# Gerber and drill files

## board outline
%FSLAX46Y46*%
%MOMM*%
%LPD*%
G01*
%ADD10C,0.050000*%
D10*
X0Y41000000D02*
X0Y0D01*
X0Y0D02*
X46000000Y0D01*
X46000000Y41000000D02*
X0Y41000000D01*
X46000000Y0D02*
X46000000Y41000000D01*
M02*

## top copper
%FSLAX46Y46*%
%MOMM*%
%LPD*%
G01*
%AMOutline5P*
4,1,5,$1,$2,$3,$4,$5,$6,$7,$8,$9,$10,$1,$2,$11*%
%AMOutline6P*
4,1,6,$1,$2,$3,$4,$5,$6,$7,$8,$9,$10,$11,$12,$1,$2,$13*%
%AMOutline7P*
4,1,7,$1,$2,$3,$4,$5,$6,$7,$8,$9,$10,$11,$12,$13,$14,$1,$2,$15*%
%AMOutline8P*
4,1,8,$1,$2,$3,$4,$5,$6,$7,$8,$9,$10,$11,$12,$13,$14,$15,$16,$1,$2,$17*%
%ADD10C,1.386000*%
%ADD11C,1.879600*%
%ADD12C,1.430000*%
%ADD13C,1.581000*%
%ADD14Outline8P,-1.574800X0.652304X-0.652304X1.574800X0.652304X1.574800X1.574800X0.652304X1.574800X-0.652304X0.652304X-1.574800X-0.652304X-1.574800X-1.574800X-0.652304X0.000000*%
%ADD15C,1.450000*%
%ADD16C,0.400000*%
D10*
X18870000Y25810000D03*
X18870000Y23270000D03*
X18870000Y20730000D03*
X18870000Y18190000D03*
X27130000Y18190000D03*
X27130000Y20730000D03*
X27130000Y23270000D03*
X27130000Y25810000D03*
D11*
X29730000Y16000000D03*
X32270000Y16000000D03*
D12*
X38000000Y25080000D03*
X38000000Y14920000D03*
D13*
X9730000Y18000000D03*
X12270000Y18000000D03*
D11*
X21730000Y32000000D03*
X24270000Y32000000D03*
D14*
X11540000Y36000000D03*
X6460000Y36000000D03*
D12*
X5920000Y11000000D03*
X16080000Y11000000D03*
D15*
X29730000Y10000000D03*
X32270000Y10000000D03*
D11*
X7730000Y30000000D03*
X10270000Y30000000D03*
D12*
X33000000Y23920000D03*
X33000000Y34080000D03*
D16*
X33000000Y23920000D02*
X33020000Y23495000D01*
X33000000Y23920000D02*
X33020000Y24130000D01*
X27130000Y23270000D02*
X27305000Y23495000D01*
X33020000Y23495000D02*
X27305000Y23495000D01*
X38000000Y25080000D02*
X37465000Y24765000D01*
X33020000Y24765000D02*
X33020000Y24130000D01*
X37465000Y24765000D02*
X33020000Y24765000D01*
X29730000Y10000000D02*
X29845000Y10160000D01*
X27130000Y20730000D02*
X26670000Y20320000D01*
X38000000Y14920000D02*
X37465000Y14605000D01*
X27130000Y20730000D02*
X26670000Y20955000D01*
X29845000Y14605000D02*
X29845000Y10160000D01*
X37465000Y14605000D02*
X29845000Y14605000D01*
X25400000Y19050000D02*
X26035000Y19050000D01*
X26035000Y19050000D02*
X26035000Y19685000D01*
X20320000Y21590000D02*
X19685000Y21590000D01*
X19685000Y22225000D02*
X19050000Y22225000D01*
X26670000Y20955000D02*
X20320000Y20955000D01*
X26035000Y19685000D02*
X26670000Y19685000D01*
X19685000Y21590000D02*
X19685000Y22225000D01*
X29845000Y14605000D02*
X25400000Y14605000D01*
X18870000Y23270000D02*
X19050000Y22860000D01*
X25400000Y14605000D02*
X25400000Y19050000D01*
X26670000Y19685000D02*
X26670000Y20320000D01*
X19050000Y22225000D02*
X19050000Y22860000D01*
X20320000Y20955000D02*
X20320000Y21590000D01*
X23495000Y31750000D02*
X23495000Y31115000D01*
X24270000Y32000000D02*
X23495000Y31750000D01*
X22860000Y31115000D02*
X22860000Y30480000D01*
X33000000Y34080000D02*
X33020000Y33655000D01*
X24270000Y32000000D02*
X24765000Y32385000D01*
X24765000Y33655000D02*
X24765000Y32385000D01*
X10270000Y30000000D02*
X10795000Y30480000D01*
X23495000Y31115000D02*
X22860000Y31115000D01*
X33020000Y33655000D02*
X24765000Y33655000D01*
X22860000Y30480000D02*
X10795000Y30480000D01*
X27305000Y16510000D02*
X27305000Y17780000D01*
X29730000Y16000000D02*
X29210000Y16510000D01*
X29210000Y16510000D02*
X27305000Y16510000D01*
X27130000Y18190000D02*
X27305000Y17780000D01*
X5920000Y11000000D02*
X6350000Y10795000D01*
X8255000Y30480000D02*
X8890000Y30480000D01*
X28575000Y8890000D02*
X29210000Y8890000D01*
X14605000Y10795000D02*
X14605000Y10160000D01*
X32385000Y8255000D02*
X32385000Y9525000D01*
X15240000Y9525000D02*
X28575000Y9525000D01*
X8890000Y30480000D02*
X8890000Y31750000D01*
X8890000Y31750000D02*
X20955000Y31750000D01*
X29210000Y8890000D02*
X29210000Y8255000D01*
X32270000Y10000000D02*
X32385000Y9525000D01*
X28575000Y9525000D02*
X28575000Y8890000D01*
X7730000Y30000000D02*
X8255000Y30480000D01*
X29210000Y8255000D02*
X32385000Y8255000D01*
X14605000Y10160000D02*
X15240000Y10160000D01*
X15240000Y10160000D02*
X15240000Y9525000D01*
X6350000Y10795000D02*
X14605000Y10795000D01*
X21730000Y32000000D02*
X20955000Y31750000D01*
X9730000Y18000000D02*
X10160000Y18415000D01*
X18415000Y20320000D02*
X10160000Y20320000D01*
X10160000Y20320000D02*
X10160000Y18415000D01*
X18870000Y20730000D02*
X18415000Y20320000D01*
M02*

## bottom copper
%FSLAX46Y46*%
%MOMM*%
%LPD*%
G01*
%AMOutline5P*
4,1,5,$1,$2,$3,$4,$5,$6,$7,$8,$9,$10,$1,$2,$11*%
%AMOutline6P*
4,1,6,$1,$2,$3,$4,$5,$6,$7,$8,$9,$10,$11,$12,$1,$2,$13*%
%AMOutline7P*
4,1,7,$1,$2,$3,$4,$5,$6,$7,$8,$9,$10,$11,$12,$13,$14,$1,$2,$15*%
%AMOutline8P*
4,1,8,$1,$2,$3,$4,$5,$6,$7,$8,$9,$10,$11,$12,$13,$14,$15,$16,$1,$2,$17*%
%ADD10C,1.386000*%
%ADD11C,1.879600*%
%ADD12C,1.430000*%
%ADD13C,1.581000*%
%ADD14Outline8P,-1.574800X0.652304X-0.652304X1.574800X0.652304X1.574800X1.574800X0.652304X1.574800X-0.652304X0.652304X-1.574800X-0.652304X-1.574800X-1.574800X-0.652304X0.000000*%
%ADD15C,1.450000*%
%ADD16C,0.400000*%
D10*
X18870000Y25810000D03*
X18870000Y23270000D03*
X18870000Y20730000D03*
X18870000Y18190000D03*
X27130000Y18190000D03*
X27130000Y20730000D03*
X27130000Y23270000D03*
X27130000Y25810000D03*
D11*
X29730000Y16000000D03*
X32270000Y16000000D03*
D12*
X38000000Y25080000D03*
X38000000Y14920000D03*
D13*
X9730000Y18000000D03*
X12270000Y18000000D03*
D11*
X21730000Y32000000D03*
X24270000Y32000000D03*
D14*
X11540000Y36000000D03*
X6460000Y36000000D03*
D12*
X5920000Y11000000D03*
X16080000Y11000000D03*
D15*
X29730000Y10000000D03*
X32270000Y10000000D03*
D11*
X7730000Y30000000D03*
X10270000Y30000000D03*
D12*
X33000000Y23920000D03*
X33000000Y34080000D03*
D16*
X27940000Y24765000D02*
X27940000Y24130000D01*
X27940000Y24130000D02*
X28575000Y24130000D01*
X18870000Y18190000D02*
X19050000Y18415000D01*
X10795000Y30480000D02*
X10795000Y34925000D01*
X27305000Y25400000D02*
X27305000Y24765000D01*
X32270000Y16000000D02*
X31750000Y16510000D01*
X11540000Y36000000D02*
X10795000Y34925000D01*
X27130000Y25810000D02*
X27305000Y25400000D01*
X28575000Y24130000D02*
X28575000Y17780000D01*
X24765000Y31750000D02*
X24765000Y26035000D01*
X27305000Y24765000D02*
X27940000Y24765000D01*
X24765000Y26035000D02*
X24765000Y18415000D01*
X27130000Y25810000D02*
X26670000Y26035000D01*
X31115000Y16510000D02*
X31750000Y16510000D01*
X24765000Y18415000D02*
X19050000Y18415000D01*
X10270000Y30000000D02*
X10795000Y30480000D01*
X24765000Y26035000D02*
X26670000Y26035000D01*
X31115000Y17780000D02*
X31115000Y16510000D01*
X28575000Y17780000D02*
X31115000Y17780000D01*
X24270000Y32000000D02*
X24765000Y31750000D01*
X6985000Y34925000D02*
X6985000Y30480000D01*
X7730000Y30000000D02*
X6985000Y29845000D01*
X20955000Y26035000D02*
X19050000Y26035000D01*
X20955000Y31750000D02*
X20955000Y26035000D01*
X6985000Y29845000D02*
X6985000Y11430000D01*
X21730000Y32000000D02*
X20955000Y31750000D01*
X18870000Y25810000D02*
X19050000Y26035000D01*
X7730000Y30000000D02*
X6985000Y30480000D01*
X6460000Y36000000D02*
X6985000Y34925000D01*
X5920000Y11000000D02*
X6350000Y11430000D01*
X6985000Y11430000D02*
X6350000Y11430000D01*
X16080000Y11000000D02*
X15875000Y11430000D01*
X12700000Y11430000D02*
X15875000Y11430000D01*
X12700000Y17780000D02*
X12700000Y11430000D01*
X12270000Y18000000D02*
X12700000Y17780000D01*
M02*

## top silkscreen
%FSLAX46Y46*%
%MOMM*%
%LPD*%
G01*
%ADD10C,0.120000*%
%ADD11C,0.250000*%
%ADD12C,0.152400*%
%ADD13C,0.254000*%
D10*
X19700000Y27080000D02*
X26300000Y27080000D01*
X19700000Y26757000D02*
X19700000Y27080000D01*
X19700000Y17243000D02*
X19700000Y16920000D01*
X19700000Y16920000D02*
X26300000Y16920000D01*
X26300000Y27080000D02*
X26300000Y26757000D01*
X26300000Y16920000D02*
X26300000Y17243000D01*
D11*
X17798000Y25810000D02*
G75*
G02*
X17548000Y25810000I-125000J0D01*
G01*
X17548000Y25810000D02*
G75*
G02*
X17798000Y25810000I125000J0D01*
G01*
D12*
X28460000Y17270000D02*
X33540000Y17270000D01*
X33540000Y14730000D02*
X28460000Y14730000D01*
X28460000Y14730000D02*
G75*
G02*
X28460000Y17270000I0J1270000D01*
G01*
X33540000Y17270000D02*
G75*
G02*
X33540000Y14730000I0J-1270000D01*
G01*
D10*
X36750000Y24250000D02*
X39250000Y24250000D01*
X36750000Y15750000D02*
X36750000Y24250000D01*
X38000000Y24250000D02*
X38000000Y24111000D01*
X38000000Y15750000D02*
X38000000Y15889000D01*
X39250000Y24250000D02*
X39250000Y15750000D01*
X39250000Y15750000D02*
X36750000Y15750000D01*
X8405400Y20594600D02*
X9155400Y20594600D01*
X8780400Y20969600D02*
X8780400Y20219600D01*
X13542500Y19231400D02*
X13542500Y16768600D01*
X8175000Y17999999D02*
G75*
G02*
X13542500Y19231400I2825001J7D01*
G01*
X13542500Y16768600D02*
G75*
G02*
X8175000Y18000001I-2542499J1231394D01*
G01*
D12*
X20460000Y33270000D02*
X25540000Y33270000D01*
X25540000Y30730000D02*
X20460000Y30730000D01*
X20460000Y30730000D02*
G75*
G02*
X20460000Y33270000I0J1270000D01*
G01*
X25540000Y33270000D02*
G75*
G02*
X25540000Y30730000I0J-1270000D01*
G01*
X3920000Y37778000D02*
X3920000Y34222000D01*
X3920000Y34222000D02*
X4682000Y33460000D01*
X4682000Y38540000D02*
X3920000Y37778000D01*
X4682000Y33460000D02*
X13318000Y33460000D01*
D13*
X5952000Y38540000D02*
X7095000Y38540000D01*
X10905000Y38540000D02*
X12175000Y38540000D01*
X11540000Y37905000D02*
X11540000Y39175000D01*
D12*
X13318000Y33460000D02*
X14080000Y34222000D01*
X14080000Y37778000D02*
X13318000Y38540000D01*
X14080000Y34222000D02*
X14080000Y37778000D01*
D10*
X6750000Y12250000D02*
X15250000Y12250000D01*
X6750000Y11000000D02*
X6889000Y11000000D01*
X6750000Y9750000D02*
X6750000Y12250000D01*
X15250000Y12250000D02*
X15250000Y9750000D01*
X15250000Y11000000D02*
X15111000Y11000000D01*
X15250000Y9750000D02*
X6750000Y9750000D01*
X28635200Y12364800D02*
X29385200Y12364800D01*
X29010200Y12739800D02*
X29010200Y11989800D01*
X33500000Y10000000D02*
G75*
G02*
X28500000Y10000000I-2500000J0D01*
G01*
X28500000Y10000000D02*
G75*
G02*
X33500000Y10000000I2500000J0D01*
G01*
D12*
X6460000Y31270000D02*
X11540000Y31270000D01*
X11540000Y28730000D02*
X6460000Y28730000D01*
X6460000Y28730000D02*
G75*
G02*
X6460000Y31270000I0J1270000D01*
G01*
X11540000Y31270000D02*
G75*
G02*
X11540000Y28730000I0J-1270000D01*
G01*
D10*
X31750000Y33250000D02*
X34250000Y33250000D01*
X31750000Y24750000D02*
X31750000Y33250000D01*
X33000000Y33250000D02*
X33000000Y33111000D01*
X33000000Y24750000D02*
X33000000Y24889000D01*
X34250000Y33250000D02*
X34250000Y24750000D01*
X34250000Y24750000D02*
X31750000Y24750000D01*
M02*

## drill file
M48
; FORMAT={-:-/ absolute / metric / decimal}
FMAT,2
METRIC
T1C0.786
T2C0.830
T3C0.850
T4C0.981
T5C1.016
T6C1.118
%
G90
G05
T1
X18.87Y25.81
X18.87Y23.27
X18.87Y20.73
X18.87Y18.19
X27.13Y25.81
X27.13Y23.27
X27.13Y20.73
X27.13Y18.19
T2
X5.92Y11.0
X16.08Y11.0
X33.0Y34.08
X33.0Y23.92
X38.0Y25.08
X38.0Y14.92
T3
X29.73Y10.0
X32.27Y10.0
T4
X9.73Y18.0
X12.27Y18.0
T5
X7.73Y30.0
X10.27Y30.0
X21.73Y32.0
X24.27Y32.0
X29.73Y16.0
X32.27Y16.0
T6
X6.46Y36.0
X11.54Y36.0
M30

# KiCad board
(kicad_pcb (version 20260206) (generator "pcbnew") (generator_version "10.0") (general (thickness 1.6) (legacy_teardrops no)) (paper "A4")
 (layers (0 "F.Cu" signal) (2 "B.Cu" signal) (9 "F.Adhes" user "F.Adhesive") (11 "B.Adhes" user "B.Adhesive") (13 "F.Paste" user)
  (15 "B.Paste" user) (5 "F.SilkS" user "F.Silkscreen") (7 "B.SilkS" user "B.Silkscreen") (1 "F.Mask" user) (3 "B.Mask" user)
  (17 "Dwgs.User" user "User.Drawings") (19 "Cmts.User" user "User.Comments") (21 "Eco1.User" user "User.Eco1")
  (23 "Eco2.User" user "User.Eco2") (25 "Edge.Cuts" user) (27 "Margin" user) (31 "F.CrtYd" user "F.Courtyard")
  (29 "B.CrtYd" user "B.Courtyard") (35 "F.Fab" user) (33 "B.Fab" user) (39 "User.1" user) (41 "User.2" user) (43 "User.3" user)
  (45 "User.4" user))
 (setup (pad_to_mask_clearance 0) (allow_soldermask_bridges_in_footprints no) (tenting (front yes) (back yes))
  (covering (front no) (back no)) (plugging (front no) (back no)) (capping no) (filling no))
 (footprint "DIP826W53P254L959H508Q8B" (layer "F.Cu") (at 23 -22)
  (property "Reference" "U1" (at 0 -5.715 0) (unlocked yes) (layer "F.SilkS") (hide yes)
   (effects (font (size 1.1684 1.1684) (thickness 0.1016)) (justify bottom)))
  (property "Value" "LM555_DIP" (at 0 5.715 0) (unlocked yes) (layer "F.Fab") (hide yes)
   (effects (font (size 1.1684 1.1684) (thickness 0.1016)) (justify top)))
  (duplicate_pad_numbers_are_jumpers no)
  (fp_line (start -3.3 -5.08) (end 3.3 -5.08) (stroke (width 0.12) (type solid)) (layer "F.SilkS"))
  (fp_line (start -3.3 -4.757) (end -3.3 -5.08) (stroke (width 0.12) (type solid)) (layer "F.SilkS"))
  (fp_line (start -3.3 4.757) (end -3.3 5.08) (stroke (width 0.12) (type solid)) (layer "F.SilkS"))
  (fp_line (start -3.3 5.08) (end 3.3 5.08) (stroke (width 0.12) (type solid)) (layer "F.SilkS"))
  (fp_line (start 3.3 -5.08) (end 3.3 -4.757) (stroke (width 0.12) (type solid)) (layer "F.SilkS"))
  (fp_line (start 3.3 5.08) (end 3.3 4.757) (stroke (width 0.12) (type solid)) (layer "F.SilkS"))
  (fp_circle (center -5.327 -3.81) (end -5.202 -3.81) (stroke (width 0.25) (type solid)) (fill yes) (layer "F.SilkS"))
  (pad "1" thru_hole circle (at -4.13 -3.81) (size 1.386 1.386) (drill 0.786) (layers "*.Cu" "*.Mask") (remove_unused_layers no) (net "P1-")
   (solder_mask_margin 0.1016) (thermal_bridge_angle 0))
  (pad "2" thru_hole circle (at -4.13 -1.27) (size 1.386 1.386) (drill 0.786) (layers "*.Cu" "*.Mask") (remove_unused_layers no)
   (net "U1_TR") (solder_mask_margin 0.1016) (thermal_bridge_angle 0))
  (pad "3" thru_hole circle (at -4.13 1.27) (size 1.386 1.386) (drill 0.786) (layers "*.Cu" "*.Mask") (remove_unused_layers no)
   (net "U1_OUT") (solder_mask_margin 0.1016) (thermal_bridge_angle 0))
  (pad "4" thru_hole circle (at -4.13 3.81) (size 1.386 1.386) (drill 0.786) (layers "*.Cu" "*.Mask") (remove_unused_layers no) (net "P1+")
   (solder_mask_margin 0.1016) (thermal_bridge_angle 0))
  (pad "5" thru_hole circle (at 4.13 3.81) (size 1.386 1.386) (drill 0.786) (layers "*.Cu" "*.Mask") (remove_unused_layers no) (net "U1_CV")
   (solder_mask_margin 0.1016) (thermal_bridge_angle 0))
  (pad "6" thru_hole circle (at 4.13 1.27) (size 1.386 1.386) (drill 0.786) (layers "*.Cu" "*.Mask") (remove_unused_layers no) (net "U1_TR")
   (solder_mask_margin 0.1016) (thermal_bridge_angle 0))
  (pad "7" thru_hole circle (at 4.13 -1.27) (size 1.386 1.386) (drill 0.786) (layers "*.Cu" "*.Mask") (remove_unused_layers no)
   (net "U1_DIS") (solder_mask_margin 0.1016) (thermal_bridge_angle 0))
  (pad "8" thru_hole circle (at 4.13 -3.81) (size 1.386 1.386) (drill 0.786) (layers "*.Cu" "*.Mask") (remove_unused_layers no) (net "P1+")
   (solder_mask_margin 0.1016) (thermal_bridge_angle 0)))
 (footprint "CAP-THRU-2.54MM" (layer "F.Cu") (at 31 -16)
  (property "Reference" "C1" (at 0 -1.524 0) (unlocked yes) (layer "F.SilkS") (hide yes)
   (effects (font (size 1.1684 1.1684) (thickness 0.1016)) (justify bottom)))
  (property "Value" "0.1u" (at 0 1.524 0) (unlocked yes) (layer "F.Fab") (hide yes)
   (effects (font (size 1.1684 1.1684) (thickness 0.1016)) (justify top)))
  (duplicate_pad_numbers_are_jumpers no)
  (fp_line (start -2.54 -1.27) (end 2.54 -1.27) (stroke (width 0.1524) (type solid)) (layer "F.SilkS"))
  (fp_line (start 2.54 1.27) (end -2.54 1.27) (stroke (width 0.1524) (type solid)) (layer "F.SilkS"))
  (fp_arc (start -2.54 1.27) (mid -3.81 0) (end -2.54 -1.27) (stroke (width 0.1524) (type solid)) (layer "F.SilkS"))
  (fp_arc (start 2.54 -1.27) (mid 3.81 0) (end 2.54 1.27) (stroke (width 0.1524) (type solid)) (layer "F.SilkS"))
  (pad "1" thru_hole circle (at -1.27 0) (size 1.8796 1.8796) (drill 1.016) (layers "*.Cu" "*.Mask") (remove_unused_layers no) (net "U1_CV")
   (solder_mask_margin 0.1016) (thermal_bridge_angle 0))
  (pad "2" thru_hole circle (at 1.27 0) (size 1.8796 1.8796) (drill 1.016) (layers "*.Cu" "*.Mask") (remove_unused_layers no) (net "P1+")
   (solder_mask_margin 0.1016) (thermal_bridge_angle 0)))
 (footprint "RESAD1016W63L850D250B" (layer "F.Cu") (at 38 -20 -90)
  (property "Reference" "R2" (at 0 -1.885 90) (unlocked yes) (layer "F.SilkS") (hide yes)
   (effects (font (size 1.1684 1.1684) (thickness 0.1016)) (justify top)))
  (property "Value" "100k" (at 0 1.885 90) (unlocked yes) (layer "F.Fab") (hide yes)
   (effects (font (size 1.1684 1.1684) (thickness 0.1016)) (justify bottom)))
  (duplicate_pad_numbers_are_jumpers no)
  (fp_line (start -4.25 1.25) (end -4.25 -1.25) (stroke (width 0.12) (type solid)) (layer "F.SilkS"))
  (fp_line (start 4.25 1.25) (end -4.25 1.25) (stroke (width 0.12) (type solid)) (layer "F.SilkS"))
  (fp_line (start -4.25 0) (end -4.111 0) (stroke (width 0.12) (type solid)) (layer "F.SilkS"))
  (fp_line (start 4.25 0) (end 4.111 0) (stroke (width 0.12) (type solid)) (layer "F.SilkS"))
  (fp_line (start -4.25 -1.25) (end 4.25 -1.25) (stroke (width 0.12) (type solid)) (layer "F.SilkS"))
  (fp_line (start 4.25 -1.25) (end 4.25 1.25) (stroke (width 0.12) (type solid)) (layer "F.SilkS"))
  (pad "1" thru_hole circle (at -5.08 0 270) (size 1.43 1.43) (drill 0.83) (layers "*.Cu" "*.Mask") (remove_unused_layers no) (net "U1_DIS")
   (solder_mask_margin 0.1016) (thermal_bridge_angle 0))
  (pad "2" thru_hole circle (at 5.08 0 270) (size 1.43 1.43) (drill 0.83) (layers "*.Cu" "*.Mask") (remove_unused_layers no) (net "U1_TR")
   (solder_mask_margin 0.1016) (thermal_bridge_angle 0)))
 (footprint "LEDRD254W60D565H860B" (layer "F.Cu") (at 11 -18)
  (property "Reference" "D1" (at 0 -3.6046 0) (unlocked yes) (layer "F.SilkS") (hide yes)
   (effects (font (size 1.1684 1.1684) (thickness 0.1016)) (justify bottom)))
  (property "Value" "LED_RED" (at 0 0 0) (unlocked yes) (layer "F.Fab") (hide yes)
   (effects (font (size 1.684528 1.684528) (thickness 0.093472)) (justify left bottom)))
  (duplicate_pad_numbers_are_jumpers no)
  (fp_line (start -2.5946 -2.5946) (end -1.8446 -2.5946) (stroke (width 0.12) (type solid)) (layer "F.SilkS"))
  (fp_line (start -2.2196 -2.9696) (end -2.2196 -2.2196) (stroke (width 0.12) (type solid)) (layer "F.SilkS"))
  (fp_line (start 2.5425 -1.2314) (end 2.5425 1.2314) (stroke (width 0.12) (type solid)) (layer "F.SilkS"))
  (fp_arc (start -2.825 0.000001) (mid -0.631694 -2.753475) (end 2.5425 -1.2314) (stroke (width 0.12) (type solid)) (layer "F.SilkS"))
  (fp_arc (start 2.5425 1.2314) (mid -0.631694 2.753475) (end -2.825 -0.000001) (stroke (width 0.12) (type solid)) (layer "F.SilkS"))
  (pad "1" thru_hole circle (at -1.27 0) (size 1.581 1.581) (drill 0.981) (layers "*.Cu" "*.Mask") (remove_unused_layers no) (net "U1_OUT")
   (solder_mask_margin 0.1016) (thermal_bridge_angle 0))
  (pad "2" thru_hole circle (at 1.27 0) (size 1.581 1.581) (drill 0.981) (layers "*.Cu" "*.Mask") (remove_unused_layers no) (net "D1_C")
   (solder_mask_margin 0.1016) (thermal_bridge_angle 0)))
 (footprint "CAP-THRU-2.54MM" (layer "F.Cu") (at 23 -32)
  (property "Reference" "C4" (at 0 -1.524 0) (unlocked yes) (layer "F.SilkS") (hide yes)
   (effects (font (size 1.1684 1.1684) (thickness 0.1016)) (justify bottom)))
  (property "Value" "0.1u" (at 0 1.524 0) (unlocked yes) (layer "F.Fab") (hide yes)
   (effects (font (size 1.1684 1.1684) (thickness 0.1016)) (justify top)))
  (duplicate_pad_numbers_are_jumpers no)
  (fp_line (start -2.54 -1.27) (end 2.54 -1.27) (stroke (width 0.1524) (type solid)) (layer "F.SilkS"))
  (fp_line (start 2.54 1.27) (end -2.54 1.27) (stroke (width 0.1524) (type solid)) (layer "F.SilkS"))
  (fp_arc (start -2.54 1.27) (mid -3.81 0) (end -2.54 -1.27) (stroke (width 0.1524) (type solid)) (layer "F.SilkS"))
  (fp_arc (start 2.54 -1.27) (mid 3.81 0) (end 2.54 1.27) (stroke (width 0.1524) (type solid)) (layer "F.SilkS"))
  (pad "1" thru_hole circle (at -1.27 0) (size 1.8796 1.8796) (drill 1.016) (layers "*.Cu" "*.Mask") (remove_unused_layers no) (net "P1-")
   (solder_mask_margin 0.1016) (thermal_bridge_angle 0))
  (pad "2" thru_hole circle (at 1.27 0) (size 1.8796 1.8796) (drill 1.016) (layers "*.Cu" "*.Mask") (remove_unused_layers no) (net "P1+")
   (solder_mask_margin 0.1016) (thermal_bridge_angle 0)))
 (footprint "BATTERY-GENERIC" (layer "F.Cu") (at 9 -36)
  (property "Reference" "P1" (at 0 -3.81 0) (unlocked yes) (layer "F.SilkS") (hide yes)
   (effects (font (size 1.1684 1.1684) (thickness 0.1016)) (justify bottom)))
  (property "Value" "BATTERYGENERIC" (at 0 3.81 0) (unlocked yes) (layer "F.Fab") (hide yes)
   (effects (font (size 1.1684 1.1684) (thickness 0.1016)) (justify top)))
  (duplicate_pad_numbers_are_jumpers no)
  (fp_line (start -5.08 -1.778) (end -5.08 1.778) (stroke (width 0.1524) (type solid)) (layer "F.SilkS"))
  (fp_line (start -5.08 1.778) (end -4.318 2.54) (stroke (width 0.1524) (type solid)) (layer "F.SilkS"))
  (fp_line (start -4.318 -2.54) (end -5.08 -1.778) (stroke (width 0.1524) (type solid)) (layer "F.SilkS"))
  (fp_line (start -4.318 2.54) (end 4.318 2.54) (stroke (width 0.1524) (type solid)) (layer "F.SilkS"))
  (fp_line (start -3.048 -2.54) (end -1.905 -2.54) (stroke (width 0.254) (type solid)) (layer "F.SilkS"))
  (fp_line (start 1.905 -2.54) (end 3.175 -2.54) (stroke (width 0.254) (type solid)) (layer "F.SilkS"))
  (fp_line (start 2.54 -1.905) (end 2.54 -3.175) (stroke (width 0.254) (type solid)) (layer "F.SilkS"))
  (fp_line (start 4.318 2.54) (end 5.08 1.778) (stroke (width 0.1524) (type solid)) (layer "F.SilkS"))
  (fp_line (start 5.08 -1.778) (end 4.318 -2.54) (stroke (width 0.1524) (type solid)) (layer "F.SilkS"))
  (fp_line (start 5.08 1.778) (end 5.08 -1.778) (stroke (width 0.1524) (type solid)) (layer "F.SilkS"))
  (pad "+" thru_hole roundrect (at 2.54 0) (size 3.1496 3.1496) (drill 1.1176) (layers "*.Cu" "*.Mask") (remove_unused_layers no)
   (roundrect_rratio 0.25) (chamfer_ratio 0.2928932188) (chamfer top_left top_right bottom_left bottom_right) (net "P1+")
   (solder_mask_margin 0.1016) (thermal_bridge_angle 0))
  (pad "-" thru_hole roundrect (at -2.54 0) (size 3.1496 3.1496) (drill 1.1176) (layers "*.Cu" "*.Mask") (remove_unused_layers no)
   (roundrect_rratio 0.25) (chamfer_ratio 0.2928932188) (chamfer top_left top_right bottom_left bottom_right) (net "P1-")
   (solder_mask_margin 0.1016) (thermal_bridge_angle 0)))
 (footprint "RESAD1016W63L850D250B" (layer "F.Cu") (at 11 -11)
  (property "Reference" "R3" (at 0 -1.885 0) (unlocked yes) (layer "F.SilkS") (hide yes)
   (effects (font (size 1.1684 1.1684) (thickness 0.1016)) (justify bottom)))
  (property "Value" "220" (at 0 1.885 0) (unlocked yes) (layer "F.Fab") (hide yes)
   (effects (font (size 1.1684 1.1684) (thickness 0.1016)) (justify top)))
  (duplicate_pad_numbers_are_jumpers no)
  (fp_line (start -4.25 -1.25) (end 4.25 -1.25) (stroke (width 0.12) (type solid)) (layer "F.SilkS"))
  (fp_line (start -4.25 0) (end -4.111 0) (stroke (width 0.12) (type solid)) (layer "F.SilkS"))
  (fp_line (start -4.25 1.25) (end -4.25 -1.25) (stroke (width 0.12) (type solid)) (layer "F.SilkS"))
  (fp_line (start 4.25 -1.25) (end 4.25 1.25) (stroke (width 0.12) (type solid)) (layer "F.SilkS"))
  (fp_line (start 4.25 0) (end 4.111 0) (stroke (width 0.12) (type solid)) (layer "F.SilkS"))
  (fp_line (start 4.25 1.25) (end -4.25 1.25) (stroke (width 0.12) (type solid)) (layer "F.SilkS"))
  (pad "1" thru_hole circle (at -5.08 0) (size 1.43 1.43) (drill 0.83) (layers "*.Cu" "*.Mask") (remove_unused_layers no) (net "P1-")
   (solder_mask_margin 0.1016) (thermal_bridge_angle 0))
  (pad "2" thru_hole circle (at 5.08 0) (size 1.43 1.43) (drill 0.83) (layers "*.Cu" "*.Mask") (remove_unused_layers no) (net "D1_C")
   (solder_mask_margin 0.1016) (thermal_bridge_angle 0)))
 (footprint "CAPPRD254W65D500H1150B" (layer "F.Cu") (at 31 -10)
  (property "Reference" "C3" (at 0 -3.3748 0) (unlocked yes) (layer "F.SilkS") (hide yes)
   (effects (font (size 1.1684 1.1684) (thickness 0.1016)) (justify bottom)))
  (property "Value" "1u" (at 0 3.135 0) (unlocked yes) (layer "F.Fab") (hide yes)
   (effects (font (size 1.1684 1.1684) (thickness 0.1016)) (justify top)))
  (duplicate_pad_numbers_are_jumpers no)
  (fp_line (start -2.3648 -2.3648) (end -1.6148 -2.3648) (stroke (width 0.12) (type solid)) (layer "F.SilkS"))
  (fp_line (start -1.9898 -2.7398) (end -1.9898 -1.9898) (stroke (width 0.12) (type solid)) (layer "F.SilkS"))
  (fp_circle (center 0 0) (end 2.5 0) (stroke (width 0.12) (type solid)) (fill no) (layer "F.SilkS"))
  (pad "1" thru_hole circle (at -1.27 0) (size 1.45 1.45) (drill 0.85) (layers "*.Cu" "*.Mask") (remove_unused_layers no) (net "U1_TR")
   (solder_mask_margin 0.1016) (thermal_bridge_angle 0))
  (pad "2" thru_hole circle (at 1.27 0) (size 1.45 1.45) (drill 0.85) (layers "*.Cu" "*.Mask") (remove_unused_layers no) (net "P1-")
   (solder_mask_margin 0.1016) (thermal_bridge_angle 0)))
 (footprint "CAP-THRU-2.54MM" (layer "F.Cu") (at 9 -30)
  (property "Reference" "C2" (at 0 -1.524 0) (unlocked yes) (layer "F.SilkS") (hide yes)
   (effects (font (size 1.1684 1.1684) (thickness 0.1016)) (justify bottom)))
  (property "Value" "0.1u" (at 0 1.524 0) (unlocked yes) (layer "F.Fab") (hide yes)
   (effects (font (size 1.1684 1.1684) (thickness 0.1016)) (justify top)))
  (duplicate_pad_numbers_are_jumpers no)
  (fp_line (start -2.54 -1.27) (end 2.54 -1.27) (stroke (width 0.1524) (type solid)) (layer "F.SilkS"))
  (fp_line (start 2.54 1.27) (end -2.54 1.27) (stroke (width 0.1524) (type solid)) (layer "F.SilkS"))
  (fp_arc (start -2.54 1.27) (mid -3.81 0) (end -2.54 -1.27) (stroke (width 0.1524) (type solid)) (layer "F.SilkS"))
  (fp_arc (start 2.54 -1.27) (mid 3.81 0) (end 2.54 1.27) (stroke (width 0.1524) (type solid)) (layer "F.SilkS"))
  (pad "1" thru_hole circle (at -1.27 0) (size 1.8796 1.8796) (drill 1.016) (layers "*.Cu" "*.Mask") (remove_unused_layers no) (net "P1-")
   (solder_mask_margin 0.1016) (thermal_bridge_angle 0))
  (pad "2" thru_hole circle (at 1.27 0) (size 1.8796 1.8796) (drill 1.016) (layers "*.Cu" "*.Mask") (remove_unused_layers no) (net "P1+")
   (solder_mask_margin 0.1016) (thermal_bridge_angle 0)))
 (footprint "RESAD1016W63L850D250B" (layer "F.Cu") (at 33 -29 90)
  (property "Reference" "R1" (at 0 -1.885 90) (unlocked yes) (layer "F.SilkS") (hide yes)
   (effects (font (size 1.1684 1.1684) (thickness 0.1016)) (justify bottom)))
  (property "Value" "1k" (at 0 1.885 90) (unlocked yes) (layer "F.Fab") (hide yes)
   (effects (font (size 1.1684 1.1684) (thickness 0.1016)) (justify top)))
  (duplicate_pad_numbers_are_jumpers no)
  (fp_line (start 4.25 -1.25) (end 4.25 1.25) (stroke (width 0.12) (type solid)) (layer "F.SilkS"))
  (fp_line (start -4.25 -1.25) (end 4.25 -1.25) (stroke (width 0.12) (type solid)) (layer "F.SilkS"))
  (fp_line (start 4.25 0) (end 4.111 0) (stroke (width 0.12) (type solid)) (layer "F.SilkS"))
  (fp_line (start -4.25 0) (end -4.111 0) (stroke (width 0.12) (type solid)) (layer "F.SilkS"))
  (fp_line (start 4.25 1.25) (end -4.25 1.25) (stroke (width 0.12) (type solid)) (layer "F.SilkS"))
  (fp_line (start -4.25 1.25) (end -4.25 -1.25) (stroke (width 0.12) (type solid)) (layer "F.SilkS"))
  (pad "1" thru_hole circle (at -5.08 0 90) (size 1.43 1.43) (drill 0.83) (layers "*.Cu" "*.Mask") (remove_unused_layers no) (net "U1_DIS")
   (solder_mask_margin 0.1016) (thermal_bridge_angle 0))
  (pad "2" thru_hole circle (at 5.08 0 90) (size 1.43 1.43) (drill 0.83) (layers "*.Cu" "*.Mask") (remove_unused_layers no) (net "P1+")
   (solder_mask_margin 0.1016) (thermal_bridge_angle 0)))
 (gr_line (start 0 -41) (end 0 0) (stroke (width 0.05) (type solid)) (layer "Edge.Cuts"))
 (gr_line (start 0 0) (end 46 0) (stroke (width 0.05) (type solid)) (layer "Edge.Cuts"))
 (gr_line (start 46 -41) (end 0 -41) (stroke (width 0.05) (type solid)) (layer "Edge.Cuts"))
 (gr_line (start 46 0) (end 46 -41) (stroke (width 0.05) (type solid)) (layer "Edge.Cuts"))
 (segment (start 33 -23.92) (end 33.02 -23.495) (width 0.4) (layer "F.Cu") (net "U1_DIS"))
 (segment (start 33 -23.92) (end 33.02 -24.13) (width 0.4) (layer "F.Cu") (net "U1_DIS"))
 (segment (start 27.13 -23.27) (end 27.305 -23.495) (width 0.4) (layer "F.Cu") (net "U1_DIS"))
 (segment (start 33.02 -23.495) (end 27.305 -23.495) (width 0.4) (layer "F.Cu") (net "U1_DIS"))
 (segment (start 38 -25.08) (end 37.465 -24.765) (width 0.4) (layer "F.Cu") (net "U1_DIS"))
 (segment (start 33.02 -24.765) (end 33.02 -24.13) (width 0.4) (layer "F.Cu") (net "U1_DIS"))
 (segment (start 37.465 -24.765) (end 33.02 -24.765) (width 0.4) (layer "F.Cu") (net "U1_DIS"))
 (segment (start 29.73 -10) (end 29.845 -10.16) (width 0.4) (layer "F.Cu") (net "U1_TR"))
 (segment (start 27.13 -20.73) (end 26.67 -20.32) (width 0.4) (layer "F.Cu") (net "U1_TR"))
 (segment (start 38 -14.92) (end 37.465 -14.605) (width 0.4) (layer "F.Cu") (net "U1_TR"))
 (segment (start 27.13 -20.73) (end 26.67 -20.955) (width 0.4) (layer "F.Cu") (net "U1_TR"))
 (segment (start 29.845 -14.605) (end 29.845 -10.16) (width 0.4) (layer "F.Cu") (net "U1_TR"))
 (segment (start 37.465 -14.605) (end 29.845 -14.605) (width 0.4) (layer "F.Cu") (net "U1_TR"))
 (segment (start 25.4 -19.05) (end 26.035 -19.05) (width 0.4) (layer "F.Cu") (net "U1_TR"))
 (segment (start 26.035 -19.05) (end 26.035 -19.685) (width 0.4) (layer "F.Cu") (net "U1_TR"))
 (segment (start 20.32 -21.59) (end 19.685 -21.59) (width 0.4) (layer "F.Cu") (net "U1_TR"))
 (segment (start 19.685 -22.225) (end 19.05 -22.225) (width 0.4) (layer "F.Cu") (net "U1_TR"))
 (segment (start 26.67 -20.955) (end 20.32 -20.955) (width 0.4) (layer "F.Cu") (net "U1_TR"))
 (segment (start 26.035 -19.685) (end 26.67 -19.685) (width 0.4) (layer "F.Cu") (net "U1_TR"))
 (segment (start 19.685 -21.59) (end 19.685 -22.225) (width 0.4) (layer "F.Cu") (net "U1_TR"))
 (segment (start 29.845 -14.605) (end 25.4 -14.605) (width 0.4) (layer "F.Cu") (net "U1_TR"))
 (segment (start 18.87 -23.27) (end 19.05 -22.86) (width 0.4) (layer "F.Cu") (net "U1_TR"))
 (segment (start 25.4 -14.605) (end 25.4 -19.05) (width 0.4) (layer "F.Cu") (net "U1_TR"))
 (segment (start 26.67 -19.685) (end 26.67 -20.32) (width 0.4) (layer "F.Cu") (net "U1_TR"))
 (segment (start 19.05 -22.225) (end 19.05 -22.86) (width 0.4) (layer "F.Cu") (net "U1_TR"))
 (segment (start 20.32 -20.955) (end 20.32 -21.59) (width 0.4) (layer "F.Cu") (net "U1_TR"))
 (segment (start 23.495 -31.75) (end 23.495 -31.115) (width 0.4) (layer "F.Cu") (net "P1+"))
 (segment (start 24.27 -32) (end 23.495 -31.75) (width 0.4) (layer "F.Cu") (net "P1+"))
 (segment (start 22.86 -31.115) (end 22.86 -30.48) (width 0.4) (layer "F.Cu") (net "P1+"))
 (segment (start 33 -34.08) (end 33.02 -33.655) (width 0.4) (layer "F.Cu") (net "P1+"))
 (segment (start 24.27 -32) (end 24.765 -32.385) (width 0.4) (layer "F.Cu") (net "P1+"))
 (segment (start 24.765 -33.655) (end 24.765 -32.385) (width 0.4) (layer "F.Cu") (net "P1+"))
 (segment (start 10.27 -30) (end 10.795 -30.48) (width 0.4) (layer "F.Cu") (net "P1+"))
 (segment (start 23.495 -31.115) (end 22.86 -31.115) (width 0.4) (layer "F.Cu") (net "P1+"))
 (segment (start 33.02 -33.655) (end 24.765 -33.655) (width 0.4) (layer "F.Cu") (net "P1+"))
 (segment (start 22.86 -30.48) (end 10.795 -30.48) (width 0.4) (layer "F.Cu") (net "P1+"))
 (segment (start 27.94 -24.765) (end 27.94 -24.13) (width 0.4) (layer "B.Cu") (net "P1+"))
 (segment (start 27.94 -24.13) (end 28.575 -24.13) (width 0.4) (layer "B.Cu") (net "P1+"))
 (segment (start 18.87 -18.19) (end 19.05 -18.415) (width 0.4) (layer "B.Cu") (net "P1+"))
 (segment (start 10.795 -30.48) (end 10.795 -34.925) (width 0.4) (layer "B.Cu") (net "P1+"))
 (segment (start 27.305 -25.4) (end 27.305 -24.765) (width 0.4) (layer "B.Cu") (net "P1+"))
 (segment (start 32.27 -16) (end 31.75 -16.51) (width 0.4) (layer "B.Cu") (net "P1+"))
 (segment (start 11.54 -36) (end 10.795 -34.925) (width 0.4) (layer "B.Cu") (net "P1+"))
 (segment (start 27.13 -25.81) (end 27.305 -25.4) (width 0.4) (layer "B.Cu") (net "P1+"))
 (segment (start 28.575 -24.13) (end 28.575 -17.78) (width 0.4) (layer "B.Cu") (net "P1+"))
 (segment (start 24.765 -31.75) (end 24.765 -26.035) (width 0.4) (layer "B.Cu") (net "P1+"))
 (segment (start 27.305 -24.765) (end 27.94 -24.765) (width 0.4) (layer "B.Cu") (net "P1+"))
 (segment (start 24.765 -26.035) (end 24.765 -18.415) (width 0.4) (layer "B.Cu") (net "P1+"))
 (segment (start 27.13 -25.81) (end 26.67 -26.035) (width 0.4) (layer "B.Cu") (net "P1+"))
 (segment (start 31.115 -16.51) (end 31.75 -16.51) (width 0.4) (layer "B.Cu") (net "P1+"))
 (segment (start 24.765 -18.415) (end 19.05 -18.415) (width 0.4) (layer "B.Cu") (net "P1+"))
 (segment (start 10.27 -30) (end 10.795 -30.48) (width 0.4) (layer "B.Cu") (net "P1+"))
 (segment (start 24.765 -26.035) (end 26.67 -26.035) (width 0.4) (layer "B.Cu") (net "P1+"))
 (segment (start 31.115 -17.78) (end 31.115 -16.51) (width 0.4) (layer "B.Cu") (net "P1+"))
 (segment (start 28.575 -17.78) (end 31.115 -17.78) (width 0.4) (layer "B.Cu") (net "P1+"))
 (segment (start 24.27 -32) (end 24.765 -31.75) (width 0.4) (layer "B.Cu") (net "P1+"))
 (segment (start 27.305 -16.51) (end 27.305 -17.78) (width 0.4) (layer "F.Cu") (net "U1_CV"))
 (segment (start 29.73 -16) (end 29.21 -16.51) (width 0.4) (layer "F.Cu") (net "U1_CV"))
 (segment (start 29.21 -16.51) (end 27.305 -16.51) (width 0.4) (layer "F.Cu") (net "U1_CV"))
 (segment (start 27.13 -18.19) (end 27.305 -17.78) (width 0.4) (layer "F.Cu") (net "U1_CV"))
 (segment (start 5.92 -11) (end 6.35 -10.795) (width 0.4) (layer "F.Cu") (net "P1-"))
 (segment (start 8.255 -30.48) (end 8.89 -30.48) (width 0.4) (layer "F.Cu") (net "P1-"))
 (segment (start 28.575 -8.89) (end 29.21 -8.89) (width 0.4) (layer "F.Cu") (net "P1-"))
 (segment (start 14.605 -10.795) (end 14.605 -10.16) (width 0.4) (layer "F.Cu") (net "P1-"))
 (segment (start 32.385 -8.255) (end 32.385 -9.525) (width 0.4) (layer "F.Cu") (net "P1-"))
 (segment (start 15.24 -9.525) (end 28.575 -9.525) (width 0.4) (layer "F.Cu") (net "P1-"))
 (segment (start 8.89 -30.48) (end 8.89 -31.75) (width 0.4) (layer "F.Cu") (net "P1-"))
 (segment (start 8.89 -31.75) (end 20.955 -31.75) (width 0.4) (layer "F.Cu") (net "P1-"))
 (segment (start 29.21 -8.89) (end 29.21 -8.255) (width 0.4) (layer "F.Cu") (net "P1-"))
 (segment (start 32.27 -10) (end 32.385 -9.525) (width 0.4) (layer "F.Cu") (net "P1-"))
 (segment (start 28.575 -9.525) (end 28.575 -8.89) (width 0.4) (layer "F.Cu") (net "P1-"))
 (segment (start 7.73 -30) (end 8.255 -30.48) (width 0.4) (layer "F.Cu") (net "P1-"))
 (segment (start 29.21 -8.255) (end 32.385 -8.255) (width 0.4) (layer "F.Cu") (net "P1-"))
 (segment (start 14.605 -10.16) (end 15.24 -10.16) (width 0.4) (layer "F.Cu") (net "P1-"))
 (segment (start 15.24 -10.16) (end 15.24 -9.525) (width 0.4) (layer "F.Cu") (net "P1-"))
 (segment (start 6.35 -10.795) (end 14.605 -10.795) (width 0.4) (layer "F.Cu") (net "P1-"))
 (segment (start 21.73 -32) (end 20.955 -31.75) (width 0.4) (layer "F.Cu") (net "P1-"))
 (segment (start 6.985 -34.925) (end 6.985 -30.48) (width 0.4) (layer "B.Cu") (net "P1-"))
 (segment (start 7.73 -30) (end 6.985 -29.845) (width 0.4) (layer "B.Cu") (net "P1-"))
 (segment (start 20.955 -26.035) (end 19.05 -26.035) (width 0.4) (layer "B.Cu") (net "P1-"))
 (segment (start 20.955 -31.75) (end 20.955 -26.035) (width 0.4) (layer "B.Cu") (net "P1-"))
 (segment (start 6.985 -29.845) (end 6.985 -11.43) (width 0.4) (layer "B.Cu") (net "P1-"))
 (segment (start 21.73 -32) (end 20.955 -31.75) (width 0.4) (layer "B.Cu") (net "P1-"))
 (segment (start 18.87 -25.81) (end 19.05 -26.035) (width 0.4) (layer "B.Cu") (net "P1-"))
 (segment (start 7.73 -30) (end 6.985 -30.48) (width 0.4) (layer "B.Cu") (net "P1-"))
 (segment (start 6.46 -36) (end 6.985 -34.925) (width 0.4) (layer "B.Cu") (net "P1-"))
 (segment (start 5.92 -11) (end 6.35 -11.43) (width 0.4) (layer "B.Cu") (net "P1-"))
 (segment (start 6.985 -11.43) (end 6.35 -11.43) (width 0.4) (layer "B.Cu") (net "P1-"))
 (segment (start 9.73 -18) (end 10.16 -18.415) (width 0.4) (layer "F.Cu") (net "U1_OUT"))
 (segment (start 18.415 -20.32) (end 10.16 -20.32) (width 0.4) (layer "F.Cu") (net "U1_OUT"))
 (segment (start 10.16 -20.32) (end 10.16 -18.415) (width 0.4) (layer "F.Cu") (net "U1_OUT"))
 (segment (start 18.87 -20.73) (end 18.415 -20.32) (width 0.4) (layer "F.Cu") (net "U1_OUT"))
 (segment (start 16.08 -11) (end 15.875 -11.43) (width 0.4) (layer "B.Cu") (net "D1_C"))
 (segment (start 12.7 -11.43) (end 15.875 -11.43) (width 0.4) (layer "B.Cu") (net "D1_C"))
 (segment (start 12.7 -17.78) (end 12.7 -11.43) (width 0.4) (layer "B.Cu") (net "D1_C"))
 (segment (start 12.27 -18) (end 12.7 -17.78) (width 0.4) (layer "B.Cu") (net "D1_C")))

